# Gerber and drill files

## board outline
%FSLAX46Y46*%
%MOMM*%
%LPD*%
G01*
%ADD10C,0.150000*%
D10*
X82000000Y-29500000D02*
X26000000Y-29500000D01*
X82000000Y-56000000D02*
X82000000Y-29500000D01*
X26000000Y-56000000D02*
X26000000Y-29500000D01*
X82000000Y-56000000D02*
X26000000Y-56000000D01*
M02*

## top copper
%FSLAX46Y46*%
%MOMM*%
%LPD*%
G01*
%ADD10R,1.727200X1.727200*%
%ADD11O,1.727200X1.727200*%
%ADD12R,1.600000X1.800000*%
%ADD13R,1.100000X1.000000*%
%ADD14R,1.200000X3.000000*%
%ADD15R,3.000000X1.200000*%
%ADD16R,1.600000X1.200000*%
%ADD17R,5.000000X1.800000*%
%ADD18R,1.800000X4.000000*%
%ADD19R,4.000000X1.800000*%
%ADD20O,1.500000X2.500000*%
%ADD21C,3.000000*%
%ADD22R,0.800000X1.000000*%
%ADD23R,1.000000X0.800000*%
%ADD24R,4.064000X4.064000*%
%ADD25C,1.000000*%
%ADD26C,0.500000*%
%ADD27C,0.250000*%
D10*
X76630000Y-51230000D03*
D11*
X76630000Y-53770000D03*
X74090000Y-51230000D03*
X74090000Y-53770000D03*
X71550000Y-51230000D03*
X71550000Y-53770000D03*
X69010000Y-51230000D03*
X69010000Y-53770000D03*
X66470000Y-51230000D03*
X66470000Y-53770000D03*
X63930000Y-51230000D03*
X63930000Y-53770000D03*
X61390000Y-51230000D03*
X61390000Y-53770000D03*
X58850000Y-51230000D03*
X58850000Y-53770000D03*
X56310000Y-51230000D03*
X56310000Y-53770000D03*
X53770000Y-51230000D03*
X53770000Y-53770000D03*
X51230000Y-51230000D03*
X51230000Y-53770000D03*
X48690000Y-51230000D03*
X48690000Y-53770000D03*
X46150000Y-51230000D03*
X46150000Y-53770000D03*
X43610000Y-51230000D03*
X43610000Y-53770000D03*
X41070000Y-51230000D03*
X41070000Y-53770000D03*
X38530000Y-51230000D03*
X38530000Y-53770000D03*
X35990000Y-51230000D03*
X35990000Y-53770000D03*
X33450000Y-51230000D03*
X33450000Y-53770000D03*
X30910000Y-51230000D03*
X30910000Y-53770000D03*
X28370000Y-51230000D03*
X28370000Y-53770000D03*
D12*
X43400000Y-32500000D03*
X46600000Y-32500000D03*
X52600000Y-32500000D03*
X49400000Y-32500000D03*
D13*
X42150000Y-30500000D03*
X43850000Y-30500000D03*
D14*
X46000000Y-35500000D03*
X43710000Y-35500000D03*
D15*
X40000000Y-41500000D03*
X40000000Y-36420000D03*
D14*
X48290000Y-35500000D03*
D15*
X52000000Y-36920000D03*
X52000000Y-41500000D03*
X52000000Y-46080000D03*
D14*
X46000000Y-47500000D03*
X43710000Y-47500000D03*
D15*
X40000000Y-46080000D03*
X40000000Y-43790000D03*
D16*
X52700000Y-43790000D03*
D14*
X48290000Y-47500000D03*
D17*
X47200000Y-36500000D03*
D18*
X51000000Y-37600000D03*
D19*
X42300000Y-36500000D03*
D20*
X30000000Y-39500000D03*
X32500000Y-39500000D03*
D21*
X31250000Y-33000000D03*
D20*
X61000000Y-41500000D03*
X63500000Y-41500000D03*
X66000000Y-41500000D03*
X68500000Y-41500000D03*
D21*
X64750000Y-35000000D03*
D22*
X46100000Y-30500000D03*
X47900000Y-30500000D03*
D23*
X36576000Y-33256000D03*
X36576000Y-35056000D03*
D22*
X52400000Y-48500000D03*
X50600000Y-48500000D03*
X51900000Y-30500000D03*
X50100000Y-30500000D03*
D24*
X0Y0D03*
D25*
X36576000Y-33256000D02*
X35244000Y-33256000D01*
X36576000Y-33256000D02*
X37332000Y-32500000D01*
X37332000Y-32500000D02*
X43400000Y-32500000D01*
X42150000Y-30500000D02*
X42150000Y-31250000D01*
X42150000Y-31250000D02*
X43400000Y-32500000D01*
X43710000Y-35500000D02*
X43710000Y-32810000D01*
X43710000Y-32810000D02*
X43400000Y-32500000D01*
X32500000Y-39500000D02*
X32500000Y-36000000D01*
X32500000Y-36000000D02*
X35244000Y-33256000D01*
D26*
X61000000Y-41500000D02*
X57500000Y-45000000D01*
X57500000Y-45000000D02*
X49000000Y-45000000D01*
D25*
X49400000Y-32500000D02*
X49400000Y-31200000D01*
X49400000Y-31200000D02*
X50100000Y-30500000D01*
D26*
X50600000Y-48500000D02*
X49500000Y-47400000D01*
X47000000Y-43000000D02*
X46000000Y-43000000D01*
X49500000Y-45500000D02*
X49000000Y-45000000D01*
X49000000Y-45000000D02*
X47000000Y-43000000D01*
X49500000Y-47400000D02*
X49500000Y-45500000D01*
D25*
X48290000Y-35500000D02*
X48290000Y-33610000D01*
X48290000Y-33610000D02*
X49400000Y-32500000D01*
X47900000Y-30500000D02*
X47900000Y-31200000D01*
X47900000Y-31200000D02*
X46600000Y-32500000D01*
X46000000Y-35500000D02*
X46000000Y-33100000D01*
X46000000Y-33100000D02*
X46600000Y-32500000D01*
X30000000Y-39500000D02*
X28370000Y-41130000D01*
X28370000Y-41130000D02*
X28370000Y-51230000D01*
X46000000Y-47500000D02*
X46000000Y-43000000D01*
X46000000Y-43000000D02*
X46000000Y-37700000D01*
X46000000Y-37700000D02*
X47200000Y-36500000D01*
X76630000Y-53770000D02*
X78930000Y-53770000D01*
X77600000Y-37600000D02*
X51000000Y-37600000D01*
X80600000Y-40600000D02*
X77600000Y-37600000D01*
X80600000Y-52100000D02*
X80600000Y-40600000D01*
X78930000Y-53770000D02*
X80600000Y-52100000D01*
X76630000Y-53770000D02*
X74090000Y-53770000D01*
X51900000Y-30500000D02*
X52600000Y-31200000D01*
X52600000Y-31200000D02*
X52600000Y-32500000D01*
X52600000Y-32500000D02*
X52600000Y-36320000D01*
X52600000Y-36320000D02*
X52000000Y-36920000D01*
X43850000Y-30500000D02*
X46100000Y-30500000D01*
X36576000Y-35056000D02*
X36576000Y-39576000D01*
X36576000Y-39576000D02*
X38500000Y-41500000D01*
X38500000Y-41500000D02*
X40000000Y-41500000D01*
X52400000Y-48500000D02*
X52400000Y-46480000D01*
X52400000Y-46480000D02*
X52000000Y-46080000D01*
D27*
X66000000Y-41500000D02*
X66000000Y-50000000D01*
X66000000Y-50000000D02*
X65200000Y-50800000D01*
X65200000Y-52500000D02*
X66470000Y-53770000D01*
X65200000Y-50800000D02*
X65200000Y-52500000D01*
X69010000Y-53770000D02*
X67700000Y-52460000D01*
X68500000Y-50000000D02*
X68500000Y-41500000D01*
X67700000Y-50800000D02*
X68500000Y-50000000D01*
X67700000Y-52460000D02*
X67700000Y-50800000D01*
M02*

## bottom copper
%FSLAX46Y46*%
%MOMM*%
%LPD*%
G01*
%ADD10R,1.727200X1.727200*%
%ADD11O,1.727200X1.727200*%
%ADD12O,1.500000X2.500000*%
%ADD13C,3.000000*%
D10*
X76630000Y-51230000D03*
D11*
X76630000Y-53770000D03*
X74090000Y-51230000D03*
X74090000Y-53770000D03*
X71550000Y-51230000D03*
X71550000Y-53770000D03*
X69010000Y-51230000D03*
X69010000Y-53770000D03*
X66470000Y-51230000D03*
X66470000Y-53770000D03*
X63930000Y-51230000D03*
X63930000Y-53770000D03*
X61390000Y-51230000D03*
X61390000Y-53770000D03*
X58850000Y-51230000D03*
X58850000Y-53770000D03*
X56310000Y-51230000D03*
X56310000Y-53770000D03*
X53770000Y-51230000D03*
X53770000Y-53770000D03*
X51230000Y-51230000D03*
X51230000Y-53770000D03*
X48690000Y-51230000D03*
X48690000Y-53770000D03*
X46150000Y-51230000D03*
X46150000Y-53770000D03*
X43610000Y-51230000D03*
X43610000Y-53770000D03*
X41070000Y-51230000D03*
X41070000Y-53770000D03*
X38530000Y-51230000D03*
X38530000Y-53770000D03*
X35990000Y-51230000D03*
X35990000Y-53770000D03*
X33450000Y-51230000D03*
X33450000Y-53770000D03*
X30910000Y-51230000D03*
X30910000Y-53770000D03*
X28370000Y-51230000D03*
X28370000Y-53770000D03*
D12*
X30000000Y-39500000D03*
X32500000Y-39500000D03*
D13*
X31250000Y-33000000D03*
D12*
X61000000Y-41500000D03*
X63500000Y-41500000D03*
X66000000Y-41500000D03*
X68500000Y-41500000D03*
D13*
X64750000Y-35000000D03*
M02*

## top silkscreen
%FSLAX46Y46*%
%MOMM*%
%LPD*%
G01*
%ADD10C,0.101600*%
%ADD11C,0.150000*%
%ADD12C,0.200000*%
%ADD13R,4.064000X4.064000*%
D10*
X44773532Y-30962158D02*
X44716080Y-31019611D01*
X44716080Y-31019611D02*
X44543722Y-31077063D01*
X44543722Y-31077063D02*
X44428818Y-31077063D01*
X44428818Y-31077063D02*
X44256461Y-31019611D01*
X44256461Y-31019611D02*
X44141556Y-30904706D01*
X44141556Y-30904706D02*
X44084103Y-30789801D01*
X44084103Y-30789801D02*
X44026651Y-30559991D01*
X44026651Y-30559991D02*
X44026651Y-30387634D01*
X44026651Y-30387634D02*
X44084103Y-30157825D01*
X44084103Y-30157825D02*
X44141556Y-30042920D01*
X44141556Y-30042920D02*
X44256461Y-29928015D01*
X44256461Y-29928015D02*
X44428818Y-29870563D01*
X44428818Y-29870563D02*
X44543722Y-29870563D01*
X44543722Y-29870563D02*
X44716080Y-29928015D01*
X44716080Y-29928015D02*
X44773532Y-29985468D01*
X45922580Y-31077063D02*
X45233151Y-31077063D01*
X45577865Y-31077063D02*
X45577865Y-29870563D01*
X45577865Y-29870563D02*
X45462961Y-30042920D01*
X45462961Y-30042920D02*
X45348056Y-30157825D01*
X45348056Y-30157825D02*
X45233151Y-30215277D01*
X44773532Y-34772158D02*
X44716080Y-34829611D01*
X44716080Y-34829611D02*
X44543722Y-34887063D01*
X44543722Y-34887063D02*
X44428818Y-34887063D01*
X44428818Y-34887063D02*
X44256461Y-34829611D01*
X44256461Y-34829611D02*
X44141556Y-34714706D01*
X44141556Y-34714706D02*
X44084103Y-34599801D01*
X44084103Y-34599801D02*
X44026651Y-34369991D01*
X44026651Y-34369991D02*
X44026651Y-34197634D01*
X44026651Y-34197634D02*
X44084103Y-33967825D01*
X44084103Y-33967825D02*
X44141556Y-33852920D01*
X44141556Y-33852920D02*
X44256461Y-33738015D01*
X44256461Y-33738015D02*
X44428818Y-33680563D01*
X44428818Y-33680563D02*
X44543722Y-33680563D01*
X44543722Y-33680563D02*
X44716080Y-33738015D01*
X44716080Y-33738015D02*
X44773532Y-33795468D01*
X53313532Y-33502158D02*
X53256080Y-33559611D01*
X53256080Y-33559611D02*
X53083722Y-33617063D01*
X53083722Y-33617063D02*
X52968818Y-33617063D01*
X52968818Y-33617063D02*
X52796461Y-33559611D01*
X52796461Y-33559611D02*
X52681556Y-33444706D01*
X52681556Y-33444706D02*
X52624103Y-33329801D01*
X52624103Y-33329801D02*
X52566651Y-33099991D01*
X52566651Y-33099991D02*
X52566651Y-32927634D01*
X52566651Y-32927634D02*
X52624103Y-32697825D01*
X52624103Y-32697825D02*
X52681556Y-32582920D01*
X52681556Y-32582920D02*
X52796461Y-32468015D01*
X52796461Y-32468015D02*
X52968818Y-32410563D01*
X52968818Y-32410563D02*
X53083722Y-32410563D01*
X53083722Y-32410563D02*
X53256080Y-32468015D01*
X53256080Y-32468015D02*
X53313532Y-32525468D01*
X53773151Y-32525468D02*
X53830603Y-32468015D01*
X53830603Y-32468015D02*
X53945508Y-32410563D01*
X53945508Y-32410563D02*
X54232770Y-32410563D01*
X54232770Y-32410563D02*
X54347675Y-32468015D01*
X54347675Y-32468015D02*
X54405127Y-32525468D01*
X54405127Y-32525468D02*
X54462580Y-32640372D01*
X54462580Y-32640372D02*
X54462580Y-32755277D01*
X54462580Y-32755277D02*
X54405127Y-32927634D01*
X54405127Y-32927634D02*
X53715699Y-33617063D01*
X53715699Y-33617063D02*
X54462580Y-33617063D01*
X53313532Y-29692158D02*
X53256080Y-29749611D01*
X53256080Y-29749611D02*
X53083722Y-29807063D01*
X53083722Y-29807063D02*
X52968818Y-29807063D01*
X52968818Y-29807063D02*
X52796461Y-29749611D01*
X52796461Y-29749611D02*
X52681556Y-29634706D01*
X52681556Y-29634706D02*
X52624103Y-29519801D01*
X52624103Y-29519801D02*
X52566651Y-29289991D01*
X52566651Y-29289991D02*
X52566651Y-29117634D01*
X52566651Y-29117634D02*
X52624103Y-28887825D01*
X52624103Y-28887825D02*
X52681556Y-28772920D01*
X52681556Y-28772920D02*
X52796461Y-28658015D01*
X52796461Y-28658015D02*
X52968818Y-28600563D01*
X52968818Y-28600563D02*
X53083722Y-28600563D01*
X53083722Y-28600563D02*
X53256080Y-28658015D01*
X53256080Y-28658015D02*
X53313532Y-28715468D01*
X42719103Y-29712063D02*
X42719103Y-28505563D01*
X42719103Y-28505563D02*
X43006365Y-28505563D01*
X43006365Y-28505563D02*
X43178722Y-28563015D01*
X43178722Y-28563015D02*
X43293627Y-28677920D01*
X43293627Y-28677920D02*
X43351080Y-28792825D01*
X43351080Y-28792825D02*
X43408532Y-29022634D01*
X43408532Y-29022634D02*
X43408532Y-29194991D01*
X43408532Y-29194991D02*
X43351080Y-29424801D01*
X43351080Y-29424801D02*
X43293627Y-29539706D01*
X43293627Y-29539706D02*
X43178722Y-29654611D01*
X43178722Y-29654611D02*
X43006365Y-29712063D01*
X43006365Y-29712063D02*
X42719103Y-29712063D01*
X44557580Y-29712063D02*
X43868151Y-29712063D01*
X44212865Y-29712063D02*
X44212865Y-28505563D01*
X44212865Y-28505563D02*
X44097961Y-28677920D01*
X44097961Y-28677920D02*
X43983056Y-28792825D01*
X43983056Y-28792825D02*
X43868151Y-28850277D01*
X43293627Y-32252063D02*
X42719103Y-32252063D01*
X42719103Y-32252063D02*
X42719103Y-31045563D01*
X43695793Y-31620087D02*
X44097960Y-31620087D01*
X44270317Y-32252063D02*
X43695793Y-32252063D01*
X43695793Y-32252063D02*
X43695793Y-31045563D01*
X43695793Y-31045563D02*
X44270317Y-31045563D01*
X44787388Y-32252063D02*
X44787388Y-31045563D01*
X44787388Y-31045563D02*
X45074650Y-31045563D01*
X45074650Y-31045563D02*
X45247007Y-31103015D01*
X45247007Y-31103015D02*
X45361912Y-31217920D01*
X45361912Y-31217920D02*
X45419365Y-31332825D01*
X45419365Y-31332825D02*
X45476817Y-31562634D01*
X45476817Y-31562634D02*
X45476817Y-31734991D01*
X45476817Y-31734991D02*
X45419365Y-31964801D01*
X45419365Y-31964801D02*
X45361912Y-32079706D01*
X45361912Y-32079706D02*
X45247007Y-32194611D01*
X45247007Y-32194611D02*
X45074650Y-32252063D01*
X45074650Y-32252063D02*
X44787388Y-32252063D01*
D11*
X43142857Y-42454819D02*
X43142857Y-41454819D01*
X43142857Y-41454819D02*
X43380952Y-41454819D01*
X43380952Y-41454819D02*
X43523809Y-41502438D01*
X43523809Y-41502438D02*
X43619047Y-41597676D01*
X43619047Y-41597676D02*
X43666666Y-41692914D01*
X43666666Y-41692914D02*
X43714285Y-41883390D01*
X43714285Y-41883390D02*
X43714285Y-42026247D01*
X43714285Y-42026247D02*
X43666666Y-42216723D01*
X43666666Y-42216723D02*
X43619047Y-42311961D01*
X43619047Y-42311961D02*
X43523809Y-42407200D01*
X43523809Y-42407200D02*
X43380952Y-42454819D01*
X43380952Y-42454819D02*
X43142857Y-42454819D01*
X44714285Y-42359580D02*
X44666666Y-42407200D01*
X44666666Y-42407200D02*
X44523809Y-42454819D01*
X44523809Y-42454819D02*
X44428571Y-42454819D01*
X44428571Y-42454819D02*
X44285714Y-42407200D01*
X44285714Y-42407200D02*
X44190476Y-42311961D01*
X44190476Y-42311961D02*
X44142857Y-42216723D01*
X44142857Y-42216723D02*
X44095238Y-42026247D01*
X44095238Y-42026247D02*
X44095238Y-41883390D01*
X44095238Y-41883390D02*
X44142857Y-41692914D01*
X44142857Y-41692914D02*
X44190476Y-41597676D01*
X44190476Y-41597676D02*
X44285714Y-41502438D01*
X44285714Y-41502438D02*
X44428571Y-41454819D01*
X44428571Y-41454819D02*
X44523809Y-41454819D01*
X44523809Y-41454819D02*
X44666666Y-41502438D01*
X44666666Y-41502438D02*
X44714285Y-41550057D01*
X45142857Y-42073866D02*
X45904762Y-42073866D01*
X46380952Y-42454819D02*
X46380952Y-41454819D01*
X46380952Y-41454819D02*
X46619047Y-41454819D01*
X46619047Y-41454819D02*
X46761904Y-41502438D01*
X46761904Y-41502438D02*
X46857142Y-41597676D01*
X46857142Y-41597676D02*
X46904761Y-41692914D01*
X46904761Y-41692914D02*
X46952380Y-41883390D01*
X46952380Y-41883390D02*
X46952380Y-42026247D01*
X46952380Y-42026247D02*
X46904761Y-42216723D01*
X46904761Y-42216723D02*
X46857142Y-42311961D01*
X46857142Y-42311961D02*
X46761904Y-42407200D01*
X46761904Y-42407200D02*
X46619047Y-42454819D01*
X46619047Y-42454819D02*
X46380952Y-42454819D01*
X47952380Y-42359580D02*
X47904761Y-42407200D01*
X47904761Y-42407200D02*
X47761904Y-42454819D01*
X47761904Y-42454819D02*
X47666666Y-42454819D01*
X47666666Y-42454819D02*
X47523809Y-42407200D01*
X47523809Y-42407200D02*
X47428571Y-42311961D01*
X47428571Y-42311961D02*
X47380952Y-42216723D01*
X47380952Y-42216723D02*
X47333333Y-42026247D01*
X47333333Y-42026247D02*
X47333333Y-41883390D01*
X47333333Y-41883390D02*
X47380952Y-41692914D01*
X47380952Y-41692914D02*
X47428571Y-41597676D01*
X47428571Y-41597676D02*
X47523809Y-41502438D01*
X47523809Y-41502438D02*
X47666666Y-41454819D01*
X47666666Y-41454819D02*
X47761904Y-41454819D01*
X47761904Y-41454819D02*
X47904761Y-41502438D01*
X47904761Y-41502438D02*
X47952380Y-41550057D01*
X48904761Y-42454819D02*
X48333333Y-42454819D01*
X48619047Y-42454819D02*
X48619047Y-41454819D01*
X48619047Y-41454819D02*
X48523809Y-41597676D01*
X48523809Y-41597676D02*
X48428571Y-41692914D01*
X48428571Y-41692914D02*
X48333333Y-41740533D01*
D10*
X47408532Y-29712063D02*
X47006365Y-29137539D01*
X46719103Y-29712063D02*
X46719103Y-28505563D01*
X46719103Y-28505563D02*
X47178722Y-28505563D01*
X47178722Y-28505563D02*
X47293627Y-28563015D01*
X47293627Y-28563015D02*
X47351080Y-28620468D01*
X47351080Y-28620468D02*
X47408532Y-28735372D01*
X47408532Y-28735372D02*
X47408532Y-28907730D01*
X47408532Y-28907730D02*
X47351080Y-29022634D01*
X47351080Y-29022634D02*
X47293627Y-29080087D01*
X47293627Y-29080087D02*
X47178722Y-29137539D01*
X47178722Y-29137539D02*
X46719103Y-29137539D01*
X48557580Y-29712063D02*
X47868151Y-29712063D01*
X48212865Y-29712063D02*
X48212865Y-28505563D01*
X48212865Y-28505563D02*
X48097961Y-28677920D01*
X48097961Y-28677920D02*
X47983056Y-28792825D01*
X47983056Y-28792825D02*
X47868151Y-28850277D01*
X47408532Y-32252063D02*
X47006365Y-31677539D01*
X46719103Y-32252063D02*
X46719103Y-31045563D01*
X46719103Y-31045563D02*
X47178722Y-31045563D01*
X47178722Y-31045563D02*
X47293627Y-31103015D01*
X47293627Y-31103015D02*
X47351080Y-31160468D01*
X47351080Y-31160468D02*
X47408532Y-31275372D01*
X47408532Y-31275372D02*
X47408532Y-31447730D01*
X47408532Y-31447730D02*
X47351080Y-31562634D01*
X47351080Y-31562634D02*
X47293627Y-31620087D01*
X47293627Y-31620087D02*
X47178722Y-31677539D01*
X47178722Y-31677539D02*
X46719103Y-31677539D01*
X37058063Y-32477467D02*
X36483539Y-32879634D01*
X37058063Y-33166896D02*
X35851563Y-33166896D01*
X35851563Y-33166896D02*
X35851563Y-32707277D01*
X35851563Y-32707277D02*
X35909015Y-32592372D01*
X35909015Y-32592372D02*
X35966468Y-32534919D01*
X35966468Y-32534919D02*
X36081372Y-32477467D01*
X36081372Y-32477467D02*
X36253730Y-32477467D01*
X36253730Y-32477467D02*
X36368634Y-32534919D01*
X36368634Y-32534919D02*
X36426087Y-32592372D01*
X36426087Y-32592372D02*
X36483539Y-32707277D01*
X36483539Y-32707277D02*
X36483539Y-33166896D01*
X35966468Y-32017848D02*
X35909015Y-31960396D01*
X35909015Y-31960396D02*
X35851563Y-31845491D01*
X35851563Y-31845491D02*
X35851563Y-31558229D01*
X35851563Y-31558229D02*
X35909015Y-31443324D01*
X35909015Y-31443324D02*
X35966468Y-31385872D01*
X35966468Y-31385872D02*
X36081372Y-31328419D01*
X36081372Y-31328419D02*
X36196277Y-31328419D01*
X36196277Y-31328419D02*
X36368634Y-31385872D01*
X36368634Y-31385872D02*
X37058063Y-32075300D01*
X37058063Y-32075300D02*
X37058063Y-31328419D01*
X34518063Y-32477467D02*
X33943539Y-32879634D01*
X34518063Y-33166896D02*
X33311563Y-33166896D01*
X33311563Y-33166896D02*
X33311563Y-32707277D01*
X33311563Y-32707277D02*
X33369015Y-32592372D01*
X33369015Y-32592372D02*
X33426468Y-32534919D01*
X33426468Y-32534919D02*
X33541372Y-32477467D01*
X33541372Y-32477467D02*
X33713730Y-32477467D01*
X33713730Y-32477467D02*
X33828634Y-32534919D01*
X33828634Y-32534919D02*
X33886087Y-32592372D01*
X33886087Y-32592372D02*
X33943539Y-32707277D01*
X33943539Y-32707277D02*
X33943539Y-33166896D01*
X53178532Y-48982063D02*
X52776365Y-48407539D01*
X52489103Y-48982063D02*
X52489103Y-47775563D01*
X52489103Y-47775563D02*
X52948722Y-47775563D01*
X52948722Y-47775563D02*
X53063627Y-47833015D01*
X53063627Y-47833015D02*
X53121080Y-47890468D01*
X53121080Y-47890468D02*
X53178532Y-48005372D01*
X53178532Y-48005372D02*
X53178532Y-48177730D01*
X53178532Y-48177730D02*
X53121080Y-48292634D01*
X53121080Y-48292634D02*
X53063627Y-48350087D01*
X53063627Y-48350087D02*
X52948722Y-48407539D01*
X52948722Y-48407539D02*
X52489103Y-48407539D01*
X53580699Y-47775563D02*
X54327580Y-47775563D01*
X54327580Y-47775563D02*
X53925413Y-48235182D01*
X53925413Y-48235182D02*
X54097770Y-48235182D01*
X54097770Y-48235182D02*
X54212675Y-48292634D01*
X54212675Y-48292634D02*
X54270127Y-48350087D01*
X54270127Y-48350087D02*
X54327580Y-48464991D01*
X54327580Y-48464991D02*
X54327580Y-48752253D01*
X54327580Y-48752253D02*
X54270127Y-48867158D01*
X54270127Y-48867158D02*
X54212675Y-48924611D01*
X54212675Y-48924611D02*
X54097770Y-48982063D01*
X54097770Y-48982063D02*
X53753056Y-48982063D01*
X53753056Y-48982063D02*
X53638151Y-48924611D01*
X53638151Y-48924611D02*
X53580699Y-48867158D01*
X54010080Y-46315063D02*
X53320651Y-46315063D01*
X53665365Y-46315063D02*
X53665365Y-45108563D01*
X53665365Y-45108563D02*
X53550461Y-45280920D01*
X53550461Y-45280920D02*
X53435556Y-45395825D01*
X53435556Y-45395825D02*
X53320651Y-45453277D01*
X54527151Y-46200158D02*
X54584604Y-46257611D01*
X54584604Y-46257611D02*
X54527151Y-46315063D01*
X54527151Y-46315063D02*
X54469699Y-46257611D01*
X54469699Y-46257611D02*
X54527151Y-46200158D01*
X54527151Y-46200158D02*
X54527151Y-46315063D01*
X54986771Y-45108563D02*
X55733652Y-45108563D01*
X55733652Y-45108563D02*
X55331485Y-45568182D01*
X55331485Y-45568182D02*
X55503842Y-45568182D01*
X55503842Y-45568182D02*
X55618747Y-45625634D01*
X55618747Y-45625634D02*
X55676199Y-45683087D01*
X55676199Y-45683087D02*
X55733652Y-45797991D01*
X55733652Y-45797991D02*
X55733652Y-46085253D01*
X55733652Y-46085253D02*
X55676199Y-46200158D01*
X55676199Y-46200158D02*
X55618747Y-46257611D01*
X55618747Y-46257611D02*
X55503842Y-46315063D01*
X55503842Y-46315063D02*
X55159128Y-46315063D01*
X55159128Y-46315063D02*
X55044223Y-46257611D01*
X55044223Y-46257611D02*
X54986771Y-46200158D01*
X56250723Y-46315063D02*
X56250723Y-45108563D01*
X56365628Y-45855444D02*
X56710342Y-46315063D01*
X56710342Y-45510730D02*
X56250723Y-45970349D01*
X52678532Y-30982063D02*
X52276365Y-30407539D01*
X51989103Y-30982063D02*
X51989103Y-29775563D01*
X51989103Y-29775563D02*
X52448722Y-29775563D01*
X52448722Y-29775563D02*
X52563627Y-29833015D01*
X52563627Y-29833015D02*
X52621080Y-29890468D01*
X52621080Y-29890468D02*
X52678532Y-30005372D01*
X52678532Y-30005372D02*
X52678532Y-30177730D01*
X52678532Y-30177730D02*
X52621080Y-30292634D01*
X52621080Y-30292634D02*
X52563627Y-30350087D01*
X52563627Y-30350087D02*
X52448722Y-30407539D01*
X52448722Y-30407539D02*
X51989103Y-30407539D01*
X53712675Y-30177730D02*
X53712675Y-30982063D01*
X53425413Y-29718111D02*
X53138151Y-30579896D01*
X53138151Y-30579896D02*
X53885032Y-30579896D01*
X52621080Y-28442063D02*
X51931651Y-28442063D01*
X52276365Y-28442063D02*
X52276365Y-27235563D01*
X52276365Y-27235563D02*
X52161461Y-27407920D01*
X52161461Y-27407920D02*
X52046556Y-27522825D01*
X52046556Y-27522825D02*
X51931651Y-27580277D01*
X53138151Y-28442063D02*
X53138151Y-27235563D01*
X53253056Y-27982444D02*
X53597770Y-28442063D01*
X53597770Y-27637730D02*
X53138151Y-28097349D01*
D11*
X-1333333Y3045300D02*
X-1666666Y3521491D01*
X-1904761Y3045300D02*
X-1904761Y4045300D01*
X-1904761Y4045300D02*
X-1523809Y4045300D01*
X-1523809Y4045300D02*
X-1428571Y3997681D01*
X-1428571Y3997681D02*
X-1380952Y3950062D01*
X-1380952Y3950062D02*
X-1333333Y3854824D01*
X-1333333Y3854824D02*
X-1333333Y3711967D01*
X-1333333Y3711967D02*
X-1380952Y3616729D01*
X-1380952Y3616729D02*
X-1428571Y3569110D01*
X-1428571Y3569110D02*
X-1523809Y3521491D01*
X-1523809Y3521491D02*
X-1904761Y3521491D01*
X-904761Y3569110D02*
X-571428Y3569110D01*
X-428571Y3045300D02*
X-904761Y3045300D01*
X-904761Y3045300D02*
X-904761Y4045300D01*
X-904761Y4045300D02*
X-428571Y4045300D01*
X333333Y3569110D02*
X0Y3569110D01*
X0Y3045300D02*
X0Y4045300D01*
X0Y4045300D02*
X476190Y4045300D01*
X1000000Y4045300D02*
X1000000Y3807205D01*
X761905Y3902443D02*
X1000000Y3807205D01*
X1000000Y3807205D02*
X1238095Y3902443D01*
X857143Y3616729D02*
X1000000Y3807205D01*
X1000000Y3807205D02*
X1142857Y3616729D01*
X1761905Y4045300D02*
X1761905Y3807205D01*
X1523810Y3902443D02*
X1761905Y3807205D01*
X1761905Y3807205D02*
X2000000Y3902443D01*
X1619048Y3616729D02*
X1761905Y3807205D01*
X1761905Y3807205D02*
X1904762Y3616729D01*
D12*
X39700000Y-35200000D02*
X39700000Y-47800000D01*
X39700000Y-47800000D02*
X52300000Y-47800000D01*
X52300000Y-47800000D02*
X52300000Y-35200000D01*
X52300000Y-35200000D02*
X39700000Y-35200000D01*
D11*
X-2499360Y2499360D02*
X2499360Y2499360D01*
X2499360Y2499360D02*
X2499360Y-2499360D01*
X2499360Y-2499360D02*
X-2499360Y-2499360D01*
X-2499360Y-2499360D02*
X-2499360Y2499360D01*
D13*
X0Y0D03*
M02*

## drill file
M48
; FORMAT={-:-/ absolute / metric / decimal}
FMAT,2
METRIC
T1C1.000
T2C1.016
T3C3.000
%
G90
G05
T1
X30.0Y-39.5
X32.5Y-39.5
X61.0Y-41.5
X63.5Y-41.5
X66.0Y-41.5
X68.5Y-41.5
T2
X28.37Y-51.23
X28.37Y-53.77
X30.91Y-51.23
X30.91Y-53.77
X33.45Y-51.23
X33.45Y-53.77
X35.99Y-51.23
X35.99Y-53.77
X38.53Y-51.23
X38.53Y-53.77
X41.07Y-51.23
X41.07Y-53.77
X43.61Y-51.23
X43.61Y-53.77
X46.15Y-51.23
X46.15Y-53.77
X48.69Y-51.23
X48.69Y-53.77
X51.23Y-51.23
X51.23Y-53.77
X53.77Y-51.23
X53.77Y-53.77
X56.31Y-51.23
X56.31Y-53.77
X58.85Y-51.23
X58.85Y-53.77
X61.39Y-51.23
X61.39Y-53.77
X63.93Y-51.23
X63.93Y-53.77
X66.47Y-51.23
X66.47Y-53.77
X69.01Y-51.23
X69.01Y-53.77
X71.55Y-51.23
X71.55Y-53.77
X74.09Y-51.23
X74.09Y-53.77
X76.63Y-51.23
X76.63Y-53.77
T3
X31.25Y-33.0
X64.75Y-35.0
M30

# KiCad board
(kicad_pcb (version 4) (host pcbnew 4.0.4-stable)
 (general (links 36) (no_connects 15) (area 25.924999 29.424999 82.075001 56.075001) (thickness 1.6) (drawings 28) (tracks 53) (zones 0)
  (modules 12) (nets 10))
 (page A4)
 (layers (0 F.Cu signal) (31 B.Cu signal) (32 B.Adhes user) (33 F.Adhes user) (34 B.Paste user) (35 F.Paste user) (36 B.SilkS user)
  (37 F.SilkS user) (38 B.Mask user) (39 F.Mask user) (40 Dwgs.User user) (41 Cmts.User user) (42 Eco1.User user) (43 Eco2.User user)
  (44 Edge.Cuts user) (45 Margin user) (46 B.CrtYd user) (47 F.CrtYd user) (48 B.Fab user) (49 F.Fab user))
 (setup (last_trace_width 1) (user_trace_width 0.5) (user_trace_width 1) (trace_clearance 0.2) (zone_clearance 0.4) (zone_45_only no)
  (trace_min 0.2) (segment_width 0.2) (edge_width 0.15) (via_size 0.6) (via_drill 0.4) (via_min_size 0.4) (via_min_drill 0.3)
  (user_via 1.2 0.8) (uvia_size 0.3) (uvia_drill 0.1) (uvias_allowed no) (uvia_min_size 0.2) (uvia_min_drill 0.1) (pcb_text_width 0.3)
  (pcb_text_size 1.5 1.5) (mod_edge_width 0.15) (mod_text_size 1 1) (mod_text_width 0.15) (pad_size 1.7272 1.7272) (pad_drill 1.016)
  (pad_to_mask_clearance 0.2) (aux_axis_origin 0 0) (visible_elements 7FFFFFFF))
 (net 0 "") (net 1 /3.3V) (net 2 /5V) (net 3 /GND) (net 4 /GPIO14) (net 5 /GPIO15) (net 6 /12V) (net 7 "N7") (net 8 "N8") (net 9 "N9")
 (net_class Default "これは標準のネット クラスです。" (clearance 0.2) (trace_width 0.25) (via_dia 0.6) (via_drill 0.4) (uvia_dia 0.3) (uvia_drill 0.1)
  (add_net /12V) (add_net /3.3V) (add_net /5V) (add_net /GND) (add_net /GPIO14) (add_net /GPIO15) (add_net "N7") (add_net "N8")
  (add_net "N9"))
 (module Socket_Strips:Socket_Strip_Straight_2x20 (layer B.Cu) (at 76.63 51.23 180)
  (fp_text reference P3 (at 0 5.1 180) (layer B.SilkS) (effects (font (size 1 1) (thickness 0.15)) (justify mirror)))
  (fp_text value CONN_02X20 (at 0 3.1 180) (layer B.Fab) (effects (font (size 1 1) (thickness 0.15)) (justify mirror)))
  (pad 1 thru_hole rect (at 0 0 180) (size 1.7272 1.7272) (drill 1.016) (layers *.Cu *.Mask B.SilkS) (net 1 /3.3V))
  (pad 2 thru_hole oval (at 0 -2.54 180) (size 1.7272 1.7272) (drill 1.016) (layers *.Cu *.Mask B.SilkS) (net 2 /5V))
  (pad 3 thru_hole oval (at 2.54 0 180) (size 1.7272 1.7272) (drill 1.016) (layers *.Cu *.Mask B.SilkS))
  (pad 4 thru_hole oval (at 2.54 -2.54 180) (size 1.7272 1.7272) (drill 1.016) (layers *.Cu *.Mask B.SilkS) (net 2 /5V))
  (pad 5 thru_hole oval (at 5.08 0 180) (size 1.7272 1.7272) (drill 1.016) (layers *.Cu *.Mask B.SilkS))
  (pad 6 thru_hole oval (at 5.08 -2.54 180) (size 1.7272 1.7272) (drill 1.016) (layers *.Cu *.Mask B.SilkS) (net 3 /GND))
  (pad 7 thru_hole oval (at 7.62 0 180) (size 1.7272 1.7272) (drill 1.016) (layers *.Cu *.Mask B.SilkS))
  (pad 8 thru_hole oval (at 7.62 -2.54 180) (size 1.7272 1.7272) (drill 1.016) (layers *.Cu *.Mask B.SilkS) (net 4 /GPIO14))
  (pad 9 thru_hole oval (at 10.16 0 180) (size 1.7272 1.7272) (drill 1.016) (layers *.Cu *.Mask B.SilkS) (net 3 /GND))
  (pad 10 thru_hole oval (at 10.16 -2.54 180) (size 1.7272 1.7272) (drill 1.016) (layers *.Cu *.Mask B.SilkS) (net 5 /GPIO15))
  (pad 11 thru_hole oval (at 12.7 0 180) (size 1.7272 1.7272) (drill 1.016) (layers *.Cu *.Mask B.SilkS))
  (pad 12 thru_hole oval (at 12.7 -2.54 180) (size 1.7272 1.7272) (drill 1.016) (layers *.Cu *.Mask B.SilkS))
  (pad 13 thru_hole oval (at 15.24 0 180) (size 1.7272 1.7272) (drill 1.016) (layers *.Cu *.Mask B.SilkS))
  (pad 14 thru_hole oval (at 15.24 -2.54 180) (size 1.7272 1.7272) (drill 1.016) (layers *.Cu *.Mask B.SilkS) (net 3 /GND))
  (pad 15 thru_hole oval (at 17.78 0 180) (size 1.7272 1.7272) (drill 1.016) (layers *.Cu *.Mask B.SilkS))
  (pad 16 thru_hole oval (at 17.78 -2.54 180) (size 1.7272 1.7272) (drill 1.016) (layers *.Cu *.Mask B.SilkS))
  (pad 17 thru_hole oval (at 20.32 0 180) (size 1.7272 1.7272) (drill 1.016) (layers *.Cu *.Mask B.SilkS) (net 1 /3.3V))
  (pad 18 thru_hole oval (at 20.32 -2.54 180) (size 1.7272 1.7272) (drill 1.016) (layers *.Cu *.Mask B.SilkS))
  (pad 19 thru_hole oval (at 22.86 0 180) (size 1.7272 1.7272) (drill 1.016) (layers *.Cu *.Mask B.SilkS))
  (pad 20 thru_hole oval (at 22.86 -2.54 180) (size 1.7272 1.7272) (drill 1.016) (layers *.Cu *.Mask B.SilkS) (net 3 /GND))
  (pad 21 thru_hole oval (at 25.4 0 180) (size 1.7272 1.7272) (drill 1.016) (layers *.Cu *.Mask B.SilkS))
  (pad 22 thru_hole oval (at 25.4 -2.54 180) (size 1.7272 1.7272) (drill 1.016) (layers *.Cu *.Mask B.SilkS))
  (pad 23 thru_hole oval (at 27.94 0 180) (size 1.7272 1.7272) (drill 1.016) (layers *.Cu *.Mask B.SilkS))
  (pad 24 thru_hole oval (at 27.94 -2.54 180) (size 1.7272 1.7272) (drill 1.016) (layers *.Cu *.Mask B.SilkS))
  (pad 25 thru_hole oval (at 30.48 0 180) (size 1.7272 1.7272) (drill 1.016) (layers *.Cu *.Mask B.SilkS) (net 3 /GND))
  (pad 26 thru_hole oval (at 30.48 -2.54 180) (size 1.7272 1.7272) (drill 1.016) (layers *.Cu *.Mask B.SilkS))
  (pad 27 thru_hole oval (at 33.02 0 180) (size 1.7272 1.7272) (drill 1.016) (layers *.Cu *.Mask B.SilkS))
  (pad 28 thru_hole oval (at 33.02 -2.54 180) (size 1.7272 1.7272) (drill 1.016) (layers *.Cu *.Mask B.SilkS))
  (pad 29 thru_hole oval (at 35.56 0 180) (size 1.7272 1.7272) (drill 1.016) (layers *.Cu *.Mask B.SilkS))
  (pad 30 thru_hole oval (at 35.56 -2.54 180) (size 1.7272 1.7272) (drill 1.016) (layers *.Cu *.Mask B.SilkS) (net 3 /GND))
  (pad 31 thru_hole oval (at 38.1 0 180) (size 1.7272 1.7272) (drill 1.016) (layers *.Cu *.Mask B.SilkS))
  (pad 32 thru_hole oval (at 38.1 -2.54 180) (size 1.7272 1.7272) (drill 1.016) (layers *.Cu *.Mask B.SilkS))
  (pad 33 thru_hole oval (at 40.64 0 180) (size 1.7272 1.7272) (drill 1.016) (layers *.Cu *.Mask B.SilkS))
  (pad 34 thru_hole oval (at 40.64 -2.54 180) (size 1.7272 1.7272) (drill 1.016) (layers *.Cu *.Mask B.SilkS) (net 3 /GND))
  (pad 35 thru_hole oval (at 43.18 0 180) (size 1.7272 1.7272) (drill 1.016) (layers *.Cu *.Mask B.SilkS))
  (pad 36 thru_hole oval (at 43.18 -2.54 180) (size 1.7272 1.7272) (drill 1.016) (layers *.Cu *.Mask B.SilkS))
  (pad 37 thru_hole oval (at 45.72 0 180) (size 1.7272 1.7272) (drill 1.016) (layers *.Cu *.Mask B.SilkS))
  (pad 38 thru_hole oval (at 45.72 -2.54 180) (size 1.7272 1.7272) (drill 1.016) (layers *.Cu *.Mask B.SilkS))
  (pad 39 thru_hole oval (at 48.26 0 180) (size 1.7272 1.7272) (drill 1.016) (layers *.Cu *.Mask B.SilkS) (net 3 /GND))
  (pad 40 thru_hole oval (at 48.26 -2.54 180) (size 1.7272 1.7272) (drill 1.016) (layers *.Cu *.Mask B.SilkS)))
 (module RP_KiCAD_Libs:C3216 (layer F.Cu) (at 45 32.5)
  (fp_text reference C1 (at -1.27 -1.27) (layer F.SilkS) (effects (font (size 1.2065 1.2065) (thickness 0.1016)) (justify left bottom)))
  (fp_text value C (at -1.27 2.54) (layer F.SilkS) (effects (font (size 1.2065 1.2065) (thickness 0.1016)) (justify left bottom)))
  (pad 1 smd rect (at -1.6 0) (size 1.6 1.8) (layers F.Cu F.Paste F.Mask) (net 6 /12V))
  (pad 2 smd rect (at 1.6 0) (size 1.6 1.8) (layers F.Cu F.Paste F.Mask) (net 3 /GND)))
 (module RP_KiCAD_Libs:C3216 (layer F.Cu) (at 51 32.5 180)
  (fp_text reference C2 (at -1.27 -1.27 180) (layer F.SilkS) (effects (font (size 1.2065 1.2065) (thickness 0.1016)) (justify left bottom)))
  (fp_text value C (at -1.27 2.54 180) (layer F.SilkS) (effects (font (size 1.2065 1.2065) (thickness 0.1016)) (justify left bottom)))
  (pad 1 smd rect (at -1.6 0 180) (size 1.6 1.8) (layers F.Cu F.Paste F.Mask) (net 2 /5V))
  (pad 2 smd rect (at 1.6 0 180) (size 1.6 1.8) (layers F.Cu F.Paste F.Mask) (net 3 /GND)))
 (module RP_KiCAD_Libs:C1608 (layer F.Cu) (at 43 30.5)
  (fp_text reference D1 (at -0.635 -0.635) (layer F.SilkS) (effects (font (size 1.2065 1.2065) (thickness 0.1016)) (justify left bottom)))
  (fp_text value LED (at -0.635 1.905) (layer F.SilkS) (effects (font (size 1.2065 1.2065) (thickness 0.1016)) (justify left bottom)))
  (pad 1 smd rect (at -0.85 0) (size 1.1 1) (layers F.Cu F.Paste F.Mask) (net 6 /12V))
  (pad 2 smd rect (at 0.85 0) (size 1.1 1) (layers F.Cu F.Paste F.Mask) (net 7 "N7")))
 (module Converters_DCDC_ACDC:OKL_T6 (layer F.Cu) (at 46 41.5)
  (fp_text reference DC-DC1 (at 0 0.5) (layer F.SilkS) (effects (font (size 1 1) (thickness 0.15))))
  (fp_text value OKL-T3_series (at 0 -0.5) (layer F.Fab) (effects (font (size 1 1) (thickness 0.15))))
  (fp_line (start -6.3 -6.3) (end -6.3 6.3) (layer F.SilkS) (width 0.2))
  (fp_line (start -6.3 6.3) (end 6.3 6.3) (layer F.SilkS) (width 0.2))
  (fp_line (start 6.3 6.3) (end 6.3 -6.3) (layer F.SilkS) (width 0.2))
  (fp_line (start 6.3 -6.3) (end -6.3 -6.3) (layer F.SilkS) (width 0.2))
  (pad 3 smd rect (at 0 -6) (size 1.2 3) (layers F.Cu F.Paste F.Mask) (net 3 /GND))
  (pad 2 smd rect (at -2.29 -6) (size 1.2 3) (layers F.Cu F.Paste F.Mask) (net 6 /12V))
  (pad 1 smd rect (at -6 0) (size 3 1.2) (layers F.Cu F.Paste F.Mask) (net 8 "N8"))
  (pad 2 smd rect (at -6 -5.08) (size 3 1.2) (layers F.Cu F.Paste F.Mask) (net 6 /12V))
  (pad 3 smd rect (at 2.29 -6) (size 1.2 3) (layers F.Cu F.Paste F.Mask) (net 3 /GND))
  (pad 4 smd rect (at 6 -4.58) (size 3 1.2) (layers F.Cu F.Paste F.Mask) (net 2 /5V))
  (pad 5 smd rect (at 6 0) (size 3 1.2) (layers F.Cu F.Paste F.Mask) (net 2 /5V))
  (pad 6 smd rect (at 6 4.58) (size 3 1.2) (layers F.Cu F.Paste F.Mask) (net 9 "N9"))
  (pad 7 smd rect (at 0 6) (size 1.2 3) (layers F.Cu F.Paste F.Mask) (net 3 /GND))
  (pad 8 smd rect (at -2.29 6) (size 1.2 3) (layers F.Cu F.Paste F.Mask))
  (pad 9 smd rect (at -6 4.58) (size 3 1.2) (layers F.Cu F.Paste F.Mask))
  (pad 10 smd rect (at -6 2.29) (size 3 1.2) (layers F.Cu F.Paste F.Mask))
  (pad 11 smd rect (at 6.7 2.29) (size 1.6 1.2) (layers F.Cu F.Paste F.Mask))
  (pad 12 smd rect (at 2.29 6) (size 1.2 3) (layers F.Cu F.Paste F.Mask))
  (pad 3 smd rect (at 1.2 -5) (size 5 1.8) (layers F.Cu F.Paste F.Mask) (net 3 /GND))
  (pad 4 smd rect (at 5 -3.9) (size 1.8 4) (layers F.Cu F.Paste F.Mask) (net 2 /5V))
  (pad 2 smd rect (at -3.7 -5) (size 4 1.8) (layers F.Cu F.Paste F.Mask) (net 6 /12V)))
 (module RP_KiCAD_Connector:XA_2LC (layer B.Cu) (at 30 39.5)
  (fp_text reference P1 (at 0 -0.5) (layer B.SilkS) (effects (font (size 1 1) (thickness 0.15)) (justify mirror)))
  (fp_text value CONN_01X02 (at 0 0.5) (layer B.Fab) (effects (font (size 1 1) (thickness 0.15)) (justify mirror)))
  (pad 1 thru_hole oval (at 0 0) (size 1.5 2.5) (drill 1) (layers *.Cu *.Mask B.SilkS) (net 3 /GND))
  (pad 2 thru_hole oval (at 2.5 0) (size 1.5 2.5) (drill 1) (layers *.Cu *.Mask B.SilkS) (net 6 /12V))
  (pad "" thru_hole circle (at 1.25 -6.5) (size 3 3) (drill 3) (layers *.Cu *.Mask B.SilkS) (clearance -0.3)))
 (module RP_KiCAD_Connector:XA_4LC (layer B.Cu) (at 61 41.5)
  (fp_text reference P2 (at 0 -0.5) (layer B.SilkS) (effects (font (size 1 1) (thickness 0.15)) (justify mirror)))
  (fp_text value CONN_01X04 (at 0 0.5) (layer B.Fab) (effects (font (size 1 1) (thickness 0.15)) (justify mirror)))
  (pad 1 thru_hole oval (at 0 0) (size 1.5 2.5) (drill 1) (layers *.Cu *.Mask B.SilkS) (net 3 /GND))
  (pad 2 thru_hole oval (at 2.5 0) (size 1.5 2.5) (drill 1) (layers *.Cu *.Mask B.SilkS))
  (pad 3 thru_hole oval (at 5 0) (size 1.5 2.5) (drill 1) (layers *.Cu *.Mask B.SilkS) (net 5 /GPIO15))
  (pad 4 thru_hole oval (at 7.5 0) (size 1.5 2.5) (drill 1) (layers *.Cu *.Mask B.SilkS) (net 4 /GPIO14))
  (pad "" thru_hole circle (at 3.75 -6.5) (size 3 3) (drill 3) (layers *.Cu *.Mask B.SilkS) (clearance -0.3)))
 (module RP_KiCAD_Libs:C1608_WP (layer F.Cu) (at 47 30.5)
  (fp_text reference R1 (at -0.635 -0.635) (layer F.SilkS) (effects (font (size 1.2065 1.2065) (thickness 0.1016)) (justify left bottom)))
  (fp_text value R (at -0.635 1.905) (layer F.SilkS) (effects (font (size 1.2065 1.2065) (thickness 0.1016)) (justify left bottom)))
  (pad 1 smd rect (at -0.9 0) (size 0.8 1) (layers F.Cu F.Paste F.Mask) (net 7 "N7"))
  (pad 2 smd rect (at 0.9 0) (size 0.8 1) (layers F.Cu F.Paste F.Mask) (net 3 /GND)))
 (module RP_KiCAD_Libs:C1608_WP (layer F.Cu) (at 36.576 34.156 270)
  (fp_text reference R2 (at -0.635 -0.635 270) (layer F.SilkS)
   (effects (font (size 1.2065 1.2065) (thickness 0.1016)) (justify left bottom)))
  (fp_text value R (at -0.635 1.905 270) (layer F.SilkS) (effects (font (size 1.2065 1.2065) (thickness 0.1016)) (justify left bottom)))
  (pad 1 smd rect (at -0.9 0 270) (size 0.8 1) (layers F.Cu F.Paste F.Mask) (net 6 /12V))
  (pad 2 smd rect (at 0.9 0 270) (size 0.8 1) (layers F.Cu F.Paste F.Mask) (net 8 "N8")))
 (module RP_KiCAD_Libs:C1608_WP (layer F.Cu) (at 51.5 48.5 180)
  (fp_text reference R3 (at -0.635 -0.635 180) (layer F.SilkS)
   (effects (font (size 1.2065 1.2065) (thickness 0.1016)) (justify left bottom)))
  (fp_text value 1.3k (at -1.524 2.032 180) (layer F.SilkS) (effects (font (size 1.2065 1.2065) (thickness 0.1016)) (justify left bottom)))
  (pad 1 smd rect (at -0.9 0 180) (size 0.8 1) (layers F.Cu F.Paste F.Mask) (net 9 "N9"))
  (pad 2 smd rect (at 0.9 0 180) (size 0.8 1) (layers F.Cu F.Paste F.Mask) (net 3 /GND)))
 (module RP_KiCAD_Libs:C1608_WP (layer F.Cu) (at 51 30.5 180)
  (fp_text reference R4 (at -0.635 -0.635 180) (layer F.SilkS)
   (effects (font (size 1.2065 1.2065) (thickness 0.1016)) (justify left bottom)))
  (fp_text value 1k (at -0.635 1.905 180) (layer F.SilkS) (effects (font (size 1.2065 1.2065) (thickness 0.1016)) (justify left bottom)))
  (pad 1 smd rect (at -0.9 0 180) (size 0.8 1) (layers F.Cu F.Paste F.Mask) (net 2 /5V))
  (pad 2 smd rect (at 0.9 0 180) (size 0.8 1) (layers F.Cu F.Paste F.Mask) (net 3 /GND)))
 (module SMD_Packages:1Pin (layer F.Cu) (at 0 0)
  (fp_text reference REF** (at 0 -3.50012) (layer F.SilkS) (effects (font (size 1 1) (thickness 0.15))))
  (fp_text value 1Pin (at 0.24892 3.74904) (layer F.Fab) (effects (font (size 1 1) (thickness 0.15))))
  (fp_line (start -2.49936 -2.49936) (end 2.49936 -2.49936) (layer F.SilkS) (width 0.15))
  (fp_line (start 2.49936 -2.49936) (end 2.49936 2.49936) (layer F.SilkS) (width 0.15))
  (fp_line (start 2.49936 2.49936) (end -2.49936 2.49936) (layer F.SilkS) (width 0.15))
  (fp_line (start -2.49936 2.49936) (end -2.49936 -2.49936) (layer F.SilkS) (width 0.15))
  (pad 1 smd rect (at 0 0) (size 4.064 4.064) (layers F.Cu F.Paste F.SilkS F.Mask)))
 (gr_line (start 82 29.5) (end 26 29.5) (angle 90) (layer Edge.Cuts) (width 0.15))
 (gr_line (start 82 56) (end 82 29.5) (angle 90) (layer Edge.Cuts) (width 0.15))
 (gr_line (start 26 56) (end 26 29.5) (angle 90) (layer Edge.Cuts) (width 0.15))
 (gr_line (start 82 56) (end 26 56) (angle 90) (layer Edge.Cuts) (width 0.15))
 (segment (start 36.576 33.256) (end 35.244 33.256) (width 1) (layer F.Cu) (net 6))
 (segment (start 36.576 33.256) (end 37.332 32.5) (width 1) (layer F.Cu) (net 6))
 (segment (start 37.332 32.5) (end 43.4 32.5) (width 1) (layer F.Cu) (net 6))
 (segment (start 42.15 30.5) (end 42.15 31.25) (width 1) (layer F.Cu) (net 6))
 (segment (start 42.15 31.25) (end 43.4 32.5) (width 1) (layer F.Cu) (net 6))
 (segment (start 43.71 35.5) (end 43.71 32.81) (width 1) (layer F.Cu) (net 6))
 (segment (start 43.71 32.81) (end 43.4 32.5) (width 1) (layer F.Cu) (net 6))
 (segment (start 32.5 39.5) (end 32.5 36) (width 1) (layer F.Cu) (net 6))
 (segment (start 32.5 36) (end 35.244 33.256) (width 1) (layer F.Cu) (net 6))
 (segment (start 61 41.5) (end 57.5 45) (width 0.5) (layer F.Cu) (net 3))
 (segment (start 57.5 45) (end 49 45) (width 0.5) (layer F.Cu) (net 3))
 (segment (start 49.4 32.5) (end 49.4 31.2) (width 1) (layer F.Cu) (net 3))
 (segment (start 49.4 31.2) (end 50.1 30.5) (width 1) (layer F.Cu) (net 3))
 (segment (start 50.6 48.5) (end 49.5 47.4) (width 0.5) (layer F.Cu) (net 3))
 (segment (start 47 43) (end 46 43) (width 0.5) (layer F.Cu) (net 3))
 (segment (start 49.5 45.5) (end 49 45) (width 0.5) (layer F.Cu) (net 3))
 (segment (start 49 45) (end 47 43) (width 0.5) (layer F.Cu) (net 3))
 (segment (start 49.5 47.4) (end 49.5 45.5) (width 0.5) (layer F.Cu) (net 3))
 (segment (start 48.29 35.5) (end 48.29 33.61) (width 1) (layer F.Cu) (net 3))
 (segment (start 48.29 33.61) (end 49.4 32.5) (width 1) (layer F.Cu) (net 3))
 (segment (start 47.9 30.5) (end 47.9 31.2) (width 1) (layer F.Cu) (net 3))
 (segment (start 47.9 31.2) (end 46.6 32.5) (width 1) (layer F.Cu) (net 3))
 (segment (start 46 35.5) (end 46 33.1) (width 1) (layer F.Cu) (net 3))
 (segment (start 46 33.1) (end 46.6 32.5) (width 1) (layer F.Cu) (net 3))
 (segment (start 30 39.5) (end 28.37 41.13) (width 1) (layer F.Cu) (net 3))
 (segment (start 28.37 41.13) (end 28.37 51.23) (width 1) (layer F.Cu) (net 3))
 (segment (start 46 47.5) (end 46 43) (width 1) (layer F.Cu) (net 3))
 (segment (start 46 43) (end 46 37.7) (width 1) (layer F.Cu) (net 3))
 (segment (start 46 37.7) (end 47.2 36.5) (width 1) (layer F.Cu) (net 3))
 (segment (start 76.63 53.77) (end 78.93 53.77) (width 1) (layer F.Cu) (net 2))
 (segment (start 77.6 37.6) (end 51 37.6) (width 1) (layer F.Cu) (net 2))
 (segment (start 80.6 40.6) (end 77.6 37.6) (width 1) (layer F.Cu) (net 2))
 (segment (start 80.6 52.1) (end 80.6 40.6) (width 1) (layer F.Cu) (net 2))
 (segment (start 78.93 53.77) (end 80.6 52.1) (width 1) (layer F.Cu) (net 2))
 (segment (start 76.63 53.77) (end 74.09 53.77) (width 1) (layer F.Cu) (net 2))
 (segment (start 51.9 30.5) (end 52.6 31.2) (width 1) (layer F.Cu) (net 2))
 (segment (start 52.6 31.2) (end 52.6 32.5) (width 1) (layer F.Cu) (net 2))
 (segment (start 52.6 32.5) (end 52.6 36.32) (width 1) (layer F.Cu) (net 2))
 (segment (start 52.6 36.32) (end 52 36.92) (width 1) (layer F.Cu) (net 2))
 (segment (start 43.85 30.5) (end 46.1 30.5) (width 1) (layer F.Cu) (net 7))
 (segment (start 36.576 35.056) (end 36.576 39.576) (width 1) (layer F.Cu) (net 8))
 (segment (start 36.576 39.576) (end 38.5 41.5) (width 1) (layer F.Cu) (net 8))
 (segment (start 38.5 41.5) (end 40 41.5) (width 1) (layer F.Cu) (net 8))
 (segment (start 52.4 48.5) (end 52.4 46.48) (width 1) (layer F.Cu) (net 9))
 (segment (start 52.4 46.48) (end 52 46.08) (width 1) (layer F.Cu) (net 9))
 (segment (start 66 41.5) (end 66 50) (width 0.25) (layer F.Cu) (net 5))
 (segment (start 66 50) (end 65.2 50.8) (width 0.25) (layer F.Cu) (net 5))
 (segment (start 65.2 52.5) (end 66.47 53.77) (width 0.25) (layer F.Cu) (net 5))
 (segment (start 65.2 50.8) (end 65.2 52.5) (width 0.25) (layer F.Cu) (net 5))
 (segment (start 69.01 53.77) (end 67.7 52.46) (width 0.25) (layer F.Cu) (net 4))
 (segment (start 68.5 50) (end 68.5 41.5) (width 0.25) (layer F.Cu) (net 4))
 (segment (start 67.7 50.8) (end 68.5 50) (width 0.25) (layer F.Cu) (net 4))
 (segment (start 67.7 52.46) (end 67.7 50.8) (width 0.25) (layer F.Cu) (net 4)))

